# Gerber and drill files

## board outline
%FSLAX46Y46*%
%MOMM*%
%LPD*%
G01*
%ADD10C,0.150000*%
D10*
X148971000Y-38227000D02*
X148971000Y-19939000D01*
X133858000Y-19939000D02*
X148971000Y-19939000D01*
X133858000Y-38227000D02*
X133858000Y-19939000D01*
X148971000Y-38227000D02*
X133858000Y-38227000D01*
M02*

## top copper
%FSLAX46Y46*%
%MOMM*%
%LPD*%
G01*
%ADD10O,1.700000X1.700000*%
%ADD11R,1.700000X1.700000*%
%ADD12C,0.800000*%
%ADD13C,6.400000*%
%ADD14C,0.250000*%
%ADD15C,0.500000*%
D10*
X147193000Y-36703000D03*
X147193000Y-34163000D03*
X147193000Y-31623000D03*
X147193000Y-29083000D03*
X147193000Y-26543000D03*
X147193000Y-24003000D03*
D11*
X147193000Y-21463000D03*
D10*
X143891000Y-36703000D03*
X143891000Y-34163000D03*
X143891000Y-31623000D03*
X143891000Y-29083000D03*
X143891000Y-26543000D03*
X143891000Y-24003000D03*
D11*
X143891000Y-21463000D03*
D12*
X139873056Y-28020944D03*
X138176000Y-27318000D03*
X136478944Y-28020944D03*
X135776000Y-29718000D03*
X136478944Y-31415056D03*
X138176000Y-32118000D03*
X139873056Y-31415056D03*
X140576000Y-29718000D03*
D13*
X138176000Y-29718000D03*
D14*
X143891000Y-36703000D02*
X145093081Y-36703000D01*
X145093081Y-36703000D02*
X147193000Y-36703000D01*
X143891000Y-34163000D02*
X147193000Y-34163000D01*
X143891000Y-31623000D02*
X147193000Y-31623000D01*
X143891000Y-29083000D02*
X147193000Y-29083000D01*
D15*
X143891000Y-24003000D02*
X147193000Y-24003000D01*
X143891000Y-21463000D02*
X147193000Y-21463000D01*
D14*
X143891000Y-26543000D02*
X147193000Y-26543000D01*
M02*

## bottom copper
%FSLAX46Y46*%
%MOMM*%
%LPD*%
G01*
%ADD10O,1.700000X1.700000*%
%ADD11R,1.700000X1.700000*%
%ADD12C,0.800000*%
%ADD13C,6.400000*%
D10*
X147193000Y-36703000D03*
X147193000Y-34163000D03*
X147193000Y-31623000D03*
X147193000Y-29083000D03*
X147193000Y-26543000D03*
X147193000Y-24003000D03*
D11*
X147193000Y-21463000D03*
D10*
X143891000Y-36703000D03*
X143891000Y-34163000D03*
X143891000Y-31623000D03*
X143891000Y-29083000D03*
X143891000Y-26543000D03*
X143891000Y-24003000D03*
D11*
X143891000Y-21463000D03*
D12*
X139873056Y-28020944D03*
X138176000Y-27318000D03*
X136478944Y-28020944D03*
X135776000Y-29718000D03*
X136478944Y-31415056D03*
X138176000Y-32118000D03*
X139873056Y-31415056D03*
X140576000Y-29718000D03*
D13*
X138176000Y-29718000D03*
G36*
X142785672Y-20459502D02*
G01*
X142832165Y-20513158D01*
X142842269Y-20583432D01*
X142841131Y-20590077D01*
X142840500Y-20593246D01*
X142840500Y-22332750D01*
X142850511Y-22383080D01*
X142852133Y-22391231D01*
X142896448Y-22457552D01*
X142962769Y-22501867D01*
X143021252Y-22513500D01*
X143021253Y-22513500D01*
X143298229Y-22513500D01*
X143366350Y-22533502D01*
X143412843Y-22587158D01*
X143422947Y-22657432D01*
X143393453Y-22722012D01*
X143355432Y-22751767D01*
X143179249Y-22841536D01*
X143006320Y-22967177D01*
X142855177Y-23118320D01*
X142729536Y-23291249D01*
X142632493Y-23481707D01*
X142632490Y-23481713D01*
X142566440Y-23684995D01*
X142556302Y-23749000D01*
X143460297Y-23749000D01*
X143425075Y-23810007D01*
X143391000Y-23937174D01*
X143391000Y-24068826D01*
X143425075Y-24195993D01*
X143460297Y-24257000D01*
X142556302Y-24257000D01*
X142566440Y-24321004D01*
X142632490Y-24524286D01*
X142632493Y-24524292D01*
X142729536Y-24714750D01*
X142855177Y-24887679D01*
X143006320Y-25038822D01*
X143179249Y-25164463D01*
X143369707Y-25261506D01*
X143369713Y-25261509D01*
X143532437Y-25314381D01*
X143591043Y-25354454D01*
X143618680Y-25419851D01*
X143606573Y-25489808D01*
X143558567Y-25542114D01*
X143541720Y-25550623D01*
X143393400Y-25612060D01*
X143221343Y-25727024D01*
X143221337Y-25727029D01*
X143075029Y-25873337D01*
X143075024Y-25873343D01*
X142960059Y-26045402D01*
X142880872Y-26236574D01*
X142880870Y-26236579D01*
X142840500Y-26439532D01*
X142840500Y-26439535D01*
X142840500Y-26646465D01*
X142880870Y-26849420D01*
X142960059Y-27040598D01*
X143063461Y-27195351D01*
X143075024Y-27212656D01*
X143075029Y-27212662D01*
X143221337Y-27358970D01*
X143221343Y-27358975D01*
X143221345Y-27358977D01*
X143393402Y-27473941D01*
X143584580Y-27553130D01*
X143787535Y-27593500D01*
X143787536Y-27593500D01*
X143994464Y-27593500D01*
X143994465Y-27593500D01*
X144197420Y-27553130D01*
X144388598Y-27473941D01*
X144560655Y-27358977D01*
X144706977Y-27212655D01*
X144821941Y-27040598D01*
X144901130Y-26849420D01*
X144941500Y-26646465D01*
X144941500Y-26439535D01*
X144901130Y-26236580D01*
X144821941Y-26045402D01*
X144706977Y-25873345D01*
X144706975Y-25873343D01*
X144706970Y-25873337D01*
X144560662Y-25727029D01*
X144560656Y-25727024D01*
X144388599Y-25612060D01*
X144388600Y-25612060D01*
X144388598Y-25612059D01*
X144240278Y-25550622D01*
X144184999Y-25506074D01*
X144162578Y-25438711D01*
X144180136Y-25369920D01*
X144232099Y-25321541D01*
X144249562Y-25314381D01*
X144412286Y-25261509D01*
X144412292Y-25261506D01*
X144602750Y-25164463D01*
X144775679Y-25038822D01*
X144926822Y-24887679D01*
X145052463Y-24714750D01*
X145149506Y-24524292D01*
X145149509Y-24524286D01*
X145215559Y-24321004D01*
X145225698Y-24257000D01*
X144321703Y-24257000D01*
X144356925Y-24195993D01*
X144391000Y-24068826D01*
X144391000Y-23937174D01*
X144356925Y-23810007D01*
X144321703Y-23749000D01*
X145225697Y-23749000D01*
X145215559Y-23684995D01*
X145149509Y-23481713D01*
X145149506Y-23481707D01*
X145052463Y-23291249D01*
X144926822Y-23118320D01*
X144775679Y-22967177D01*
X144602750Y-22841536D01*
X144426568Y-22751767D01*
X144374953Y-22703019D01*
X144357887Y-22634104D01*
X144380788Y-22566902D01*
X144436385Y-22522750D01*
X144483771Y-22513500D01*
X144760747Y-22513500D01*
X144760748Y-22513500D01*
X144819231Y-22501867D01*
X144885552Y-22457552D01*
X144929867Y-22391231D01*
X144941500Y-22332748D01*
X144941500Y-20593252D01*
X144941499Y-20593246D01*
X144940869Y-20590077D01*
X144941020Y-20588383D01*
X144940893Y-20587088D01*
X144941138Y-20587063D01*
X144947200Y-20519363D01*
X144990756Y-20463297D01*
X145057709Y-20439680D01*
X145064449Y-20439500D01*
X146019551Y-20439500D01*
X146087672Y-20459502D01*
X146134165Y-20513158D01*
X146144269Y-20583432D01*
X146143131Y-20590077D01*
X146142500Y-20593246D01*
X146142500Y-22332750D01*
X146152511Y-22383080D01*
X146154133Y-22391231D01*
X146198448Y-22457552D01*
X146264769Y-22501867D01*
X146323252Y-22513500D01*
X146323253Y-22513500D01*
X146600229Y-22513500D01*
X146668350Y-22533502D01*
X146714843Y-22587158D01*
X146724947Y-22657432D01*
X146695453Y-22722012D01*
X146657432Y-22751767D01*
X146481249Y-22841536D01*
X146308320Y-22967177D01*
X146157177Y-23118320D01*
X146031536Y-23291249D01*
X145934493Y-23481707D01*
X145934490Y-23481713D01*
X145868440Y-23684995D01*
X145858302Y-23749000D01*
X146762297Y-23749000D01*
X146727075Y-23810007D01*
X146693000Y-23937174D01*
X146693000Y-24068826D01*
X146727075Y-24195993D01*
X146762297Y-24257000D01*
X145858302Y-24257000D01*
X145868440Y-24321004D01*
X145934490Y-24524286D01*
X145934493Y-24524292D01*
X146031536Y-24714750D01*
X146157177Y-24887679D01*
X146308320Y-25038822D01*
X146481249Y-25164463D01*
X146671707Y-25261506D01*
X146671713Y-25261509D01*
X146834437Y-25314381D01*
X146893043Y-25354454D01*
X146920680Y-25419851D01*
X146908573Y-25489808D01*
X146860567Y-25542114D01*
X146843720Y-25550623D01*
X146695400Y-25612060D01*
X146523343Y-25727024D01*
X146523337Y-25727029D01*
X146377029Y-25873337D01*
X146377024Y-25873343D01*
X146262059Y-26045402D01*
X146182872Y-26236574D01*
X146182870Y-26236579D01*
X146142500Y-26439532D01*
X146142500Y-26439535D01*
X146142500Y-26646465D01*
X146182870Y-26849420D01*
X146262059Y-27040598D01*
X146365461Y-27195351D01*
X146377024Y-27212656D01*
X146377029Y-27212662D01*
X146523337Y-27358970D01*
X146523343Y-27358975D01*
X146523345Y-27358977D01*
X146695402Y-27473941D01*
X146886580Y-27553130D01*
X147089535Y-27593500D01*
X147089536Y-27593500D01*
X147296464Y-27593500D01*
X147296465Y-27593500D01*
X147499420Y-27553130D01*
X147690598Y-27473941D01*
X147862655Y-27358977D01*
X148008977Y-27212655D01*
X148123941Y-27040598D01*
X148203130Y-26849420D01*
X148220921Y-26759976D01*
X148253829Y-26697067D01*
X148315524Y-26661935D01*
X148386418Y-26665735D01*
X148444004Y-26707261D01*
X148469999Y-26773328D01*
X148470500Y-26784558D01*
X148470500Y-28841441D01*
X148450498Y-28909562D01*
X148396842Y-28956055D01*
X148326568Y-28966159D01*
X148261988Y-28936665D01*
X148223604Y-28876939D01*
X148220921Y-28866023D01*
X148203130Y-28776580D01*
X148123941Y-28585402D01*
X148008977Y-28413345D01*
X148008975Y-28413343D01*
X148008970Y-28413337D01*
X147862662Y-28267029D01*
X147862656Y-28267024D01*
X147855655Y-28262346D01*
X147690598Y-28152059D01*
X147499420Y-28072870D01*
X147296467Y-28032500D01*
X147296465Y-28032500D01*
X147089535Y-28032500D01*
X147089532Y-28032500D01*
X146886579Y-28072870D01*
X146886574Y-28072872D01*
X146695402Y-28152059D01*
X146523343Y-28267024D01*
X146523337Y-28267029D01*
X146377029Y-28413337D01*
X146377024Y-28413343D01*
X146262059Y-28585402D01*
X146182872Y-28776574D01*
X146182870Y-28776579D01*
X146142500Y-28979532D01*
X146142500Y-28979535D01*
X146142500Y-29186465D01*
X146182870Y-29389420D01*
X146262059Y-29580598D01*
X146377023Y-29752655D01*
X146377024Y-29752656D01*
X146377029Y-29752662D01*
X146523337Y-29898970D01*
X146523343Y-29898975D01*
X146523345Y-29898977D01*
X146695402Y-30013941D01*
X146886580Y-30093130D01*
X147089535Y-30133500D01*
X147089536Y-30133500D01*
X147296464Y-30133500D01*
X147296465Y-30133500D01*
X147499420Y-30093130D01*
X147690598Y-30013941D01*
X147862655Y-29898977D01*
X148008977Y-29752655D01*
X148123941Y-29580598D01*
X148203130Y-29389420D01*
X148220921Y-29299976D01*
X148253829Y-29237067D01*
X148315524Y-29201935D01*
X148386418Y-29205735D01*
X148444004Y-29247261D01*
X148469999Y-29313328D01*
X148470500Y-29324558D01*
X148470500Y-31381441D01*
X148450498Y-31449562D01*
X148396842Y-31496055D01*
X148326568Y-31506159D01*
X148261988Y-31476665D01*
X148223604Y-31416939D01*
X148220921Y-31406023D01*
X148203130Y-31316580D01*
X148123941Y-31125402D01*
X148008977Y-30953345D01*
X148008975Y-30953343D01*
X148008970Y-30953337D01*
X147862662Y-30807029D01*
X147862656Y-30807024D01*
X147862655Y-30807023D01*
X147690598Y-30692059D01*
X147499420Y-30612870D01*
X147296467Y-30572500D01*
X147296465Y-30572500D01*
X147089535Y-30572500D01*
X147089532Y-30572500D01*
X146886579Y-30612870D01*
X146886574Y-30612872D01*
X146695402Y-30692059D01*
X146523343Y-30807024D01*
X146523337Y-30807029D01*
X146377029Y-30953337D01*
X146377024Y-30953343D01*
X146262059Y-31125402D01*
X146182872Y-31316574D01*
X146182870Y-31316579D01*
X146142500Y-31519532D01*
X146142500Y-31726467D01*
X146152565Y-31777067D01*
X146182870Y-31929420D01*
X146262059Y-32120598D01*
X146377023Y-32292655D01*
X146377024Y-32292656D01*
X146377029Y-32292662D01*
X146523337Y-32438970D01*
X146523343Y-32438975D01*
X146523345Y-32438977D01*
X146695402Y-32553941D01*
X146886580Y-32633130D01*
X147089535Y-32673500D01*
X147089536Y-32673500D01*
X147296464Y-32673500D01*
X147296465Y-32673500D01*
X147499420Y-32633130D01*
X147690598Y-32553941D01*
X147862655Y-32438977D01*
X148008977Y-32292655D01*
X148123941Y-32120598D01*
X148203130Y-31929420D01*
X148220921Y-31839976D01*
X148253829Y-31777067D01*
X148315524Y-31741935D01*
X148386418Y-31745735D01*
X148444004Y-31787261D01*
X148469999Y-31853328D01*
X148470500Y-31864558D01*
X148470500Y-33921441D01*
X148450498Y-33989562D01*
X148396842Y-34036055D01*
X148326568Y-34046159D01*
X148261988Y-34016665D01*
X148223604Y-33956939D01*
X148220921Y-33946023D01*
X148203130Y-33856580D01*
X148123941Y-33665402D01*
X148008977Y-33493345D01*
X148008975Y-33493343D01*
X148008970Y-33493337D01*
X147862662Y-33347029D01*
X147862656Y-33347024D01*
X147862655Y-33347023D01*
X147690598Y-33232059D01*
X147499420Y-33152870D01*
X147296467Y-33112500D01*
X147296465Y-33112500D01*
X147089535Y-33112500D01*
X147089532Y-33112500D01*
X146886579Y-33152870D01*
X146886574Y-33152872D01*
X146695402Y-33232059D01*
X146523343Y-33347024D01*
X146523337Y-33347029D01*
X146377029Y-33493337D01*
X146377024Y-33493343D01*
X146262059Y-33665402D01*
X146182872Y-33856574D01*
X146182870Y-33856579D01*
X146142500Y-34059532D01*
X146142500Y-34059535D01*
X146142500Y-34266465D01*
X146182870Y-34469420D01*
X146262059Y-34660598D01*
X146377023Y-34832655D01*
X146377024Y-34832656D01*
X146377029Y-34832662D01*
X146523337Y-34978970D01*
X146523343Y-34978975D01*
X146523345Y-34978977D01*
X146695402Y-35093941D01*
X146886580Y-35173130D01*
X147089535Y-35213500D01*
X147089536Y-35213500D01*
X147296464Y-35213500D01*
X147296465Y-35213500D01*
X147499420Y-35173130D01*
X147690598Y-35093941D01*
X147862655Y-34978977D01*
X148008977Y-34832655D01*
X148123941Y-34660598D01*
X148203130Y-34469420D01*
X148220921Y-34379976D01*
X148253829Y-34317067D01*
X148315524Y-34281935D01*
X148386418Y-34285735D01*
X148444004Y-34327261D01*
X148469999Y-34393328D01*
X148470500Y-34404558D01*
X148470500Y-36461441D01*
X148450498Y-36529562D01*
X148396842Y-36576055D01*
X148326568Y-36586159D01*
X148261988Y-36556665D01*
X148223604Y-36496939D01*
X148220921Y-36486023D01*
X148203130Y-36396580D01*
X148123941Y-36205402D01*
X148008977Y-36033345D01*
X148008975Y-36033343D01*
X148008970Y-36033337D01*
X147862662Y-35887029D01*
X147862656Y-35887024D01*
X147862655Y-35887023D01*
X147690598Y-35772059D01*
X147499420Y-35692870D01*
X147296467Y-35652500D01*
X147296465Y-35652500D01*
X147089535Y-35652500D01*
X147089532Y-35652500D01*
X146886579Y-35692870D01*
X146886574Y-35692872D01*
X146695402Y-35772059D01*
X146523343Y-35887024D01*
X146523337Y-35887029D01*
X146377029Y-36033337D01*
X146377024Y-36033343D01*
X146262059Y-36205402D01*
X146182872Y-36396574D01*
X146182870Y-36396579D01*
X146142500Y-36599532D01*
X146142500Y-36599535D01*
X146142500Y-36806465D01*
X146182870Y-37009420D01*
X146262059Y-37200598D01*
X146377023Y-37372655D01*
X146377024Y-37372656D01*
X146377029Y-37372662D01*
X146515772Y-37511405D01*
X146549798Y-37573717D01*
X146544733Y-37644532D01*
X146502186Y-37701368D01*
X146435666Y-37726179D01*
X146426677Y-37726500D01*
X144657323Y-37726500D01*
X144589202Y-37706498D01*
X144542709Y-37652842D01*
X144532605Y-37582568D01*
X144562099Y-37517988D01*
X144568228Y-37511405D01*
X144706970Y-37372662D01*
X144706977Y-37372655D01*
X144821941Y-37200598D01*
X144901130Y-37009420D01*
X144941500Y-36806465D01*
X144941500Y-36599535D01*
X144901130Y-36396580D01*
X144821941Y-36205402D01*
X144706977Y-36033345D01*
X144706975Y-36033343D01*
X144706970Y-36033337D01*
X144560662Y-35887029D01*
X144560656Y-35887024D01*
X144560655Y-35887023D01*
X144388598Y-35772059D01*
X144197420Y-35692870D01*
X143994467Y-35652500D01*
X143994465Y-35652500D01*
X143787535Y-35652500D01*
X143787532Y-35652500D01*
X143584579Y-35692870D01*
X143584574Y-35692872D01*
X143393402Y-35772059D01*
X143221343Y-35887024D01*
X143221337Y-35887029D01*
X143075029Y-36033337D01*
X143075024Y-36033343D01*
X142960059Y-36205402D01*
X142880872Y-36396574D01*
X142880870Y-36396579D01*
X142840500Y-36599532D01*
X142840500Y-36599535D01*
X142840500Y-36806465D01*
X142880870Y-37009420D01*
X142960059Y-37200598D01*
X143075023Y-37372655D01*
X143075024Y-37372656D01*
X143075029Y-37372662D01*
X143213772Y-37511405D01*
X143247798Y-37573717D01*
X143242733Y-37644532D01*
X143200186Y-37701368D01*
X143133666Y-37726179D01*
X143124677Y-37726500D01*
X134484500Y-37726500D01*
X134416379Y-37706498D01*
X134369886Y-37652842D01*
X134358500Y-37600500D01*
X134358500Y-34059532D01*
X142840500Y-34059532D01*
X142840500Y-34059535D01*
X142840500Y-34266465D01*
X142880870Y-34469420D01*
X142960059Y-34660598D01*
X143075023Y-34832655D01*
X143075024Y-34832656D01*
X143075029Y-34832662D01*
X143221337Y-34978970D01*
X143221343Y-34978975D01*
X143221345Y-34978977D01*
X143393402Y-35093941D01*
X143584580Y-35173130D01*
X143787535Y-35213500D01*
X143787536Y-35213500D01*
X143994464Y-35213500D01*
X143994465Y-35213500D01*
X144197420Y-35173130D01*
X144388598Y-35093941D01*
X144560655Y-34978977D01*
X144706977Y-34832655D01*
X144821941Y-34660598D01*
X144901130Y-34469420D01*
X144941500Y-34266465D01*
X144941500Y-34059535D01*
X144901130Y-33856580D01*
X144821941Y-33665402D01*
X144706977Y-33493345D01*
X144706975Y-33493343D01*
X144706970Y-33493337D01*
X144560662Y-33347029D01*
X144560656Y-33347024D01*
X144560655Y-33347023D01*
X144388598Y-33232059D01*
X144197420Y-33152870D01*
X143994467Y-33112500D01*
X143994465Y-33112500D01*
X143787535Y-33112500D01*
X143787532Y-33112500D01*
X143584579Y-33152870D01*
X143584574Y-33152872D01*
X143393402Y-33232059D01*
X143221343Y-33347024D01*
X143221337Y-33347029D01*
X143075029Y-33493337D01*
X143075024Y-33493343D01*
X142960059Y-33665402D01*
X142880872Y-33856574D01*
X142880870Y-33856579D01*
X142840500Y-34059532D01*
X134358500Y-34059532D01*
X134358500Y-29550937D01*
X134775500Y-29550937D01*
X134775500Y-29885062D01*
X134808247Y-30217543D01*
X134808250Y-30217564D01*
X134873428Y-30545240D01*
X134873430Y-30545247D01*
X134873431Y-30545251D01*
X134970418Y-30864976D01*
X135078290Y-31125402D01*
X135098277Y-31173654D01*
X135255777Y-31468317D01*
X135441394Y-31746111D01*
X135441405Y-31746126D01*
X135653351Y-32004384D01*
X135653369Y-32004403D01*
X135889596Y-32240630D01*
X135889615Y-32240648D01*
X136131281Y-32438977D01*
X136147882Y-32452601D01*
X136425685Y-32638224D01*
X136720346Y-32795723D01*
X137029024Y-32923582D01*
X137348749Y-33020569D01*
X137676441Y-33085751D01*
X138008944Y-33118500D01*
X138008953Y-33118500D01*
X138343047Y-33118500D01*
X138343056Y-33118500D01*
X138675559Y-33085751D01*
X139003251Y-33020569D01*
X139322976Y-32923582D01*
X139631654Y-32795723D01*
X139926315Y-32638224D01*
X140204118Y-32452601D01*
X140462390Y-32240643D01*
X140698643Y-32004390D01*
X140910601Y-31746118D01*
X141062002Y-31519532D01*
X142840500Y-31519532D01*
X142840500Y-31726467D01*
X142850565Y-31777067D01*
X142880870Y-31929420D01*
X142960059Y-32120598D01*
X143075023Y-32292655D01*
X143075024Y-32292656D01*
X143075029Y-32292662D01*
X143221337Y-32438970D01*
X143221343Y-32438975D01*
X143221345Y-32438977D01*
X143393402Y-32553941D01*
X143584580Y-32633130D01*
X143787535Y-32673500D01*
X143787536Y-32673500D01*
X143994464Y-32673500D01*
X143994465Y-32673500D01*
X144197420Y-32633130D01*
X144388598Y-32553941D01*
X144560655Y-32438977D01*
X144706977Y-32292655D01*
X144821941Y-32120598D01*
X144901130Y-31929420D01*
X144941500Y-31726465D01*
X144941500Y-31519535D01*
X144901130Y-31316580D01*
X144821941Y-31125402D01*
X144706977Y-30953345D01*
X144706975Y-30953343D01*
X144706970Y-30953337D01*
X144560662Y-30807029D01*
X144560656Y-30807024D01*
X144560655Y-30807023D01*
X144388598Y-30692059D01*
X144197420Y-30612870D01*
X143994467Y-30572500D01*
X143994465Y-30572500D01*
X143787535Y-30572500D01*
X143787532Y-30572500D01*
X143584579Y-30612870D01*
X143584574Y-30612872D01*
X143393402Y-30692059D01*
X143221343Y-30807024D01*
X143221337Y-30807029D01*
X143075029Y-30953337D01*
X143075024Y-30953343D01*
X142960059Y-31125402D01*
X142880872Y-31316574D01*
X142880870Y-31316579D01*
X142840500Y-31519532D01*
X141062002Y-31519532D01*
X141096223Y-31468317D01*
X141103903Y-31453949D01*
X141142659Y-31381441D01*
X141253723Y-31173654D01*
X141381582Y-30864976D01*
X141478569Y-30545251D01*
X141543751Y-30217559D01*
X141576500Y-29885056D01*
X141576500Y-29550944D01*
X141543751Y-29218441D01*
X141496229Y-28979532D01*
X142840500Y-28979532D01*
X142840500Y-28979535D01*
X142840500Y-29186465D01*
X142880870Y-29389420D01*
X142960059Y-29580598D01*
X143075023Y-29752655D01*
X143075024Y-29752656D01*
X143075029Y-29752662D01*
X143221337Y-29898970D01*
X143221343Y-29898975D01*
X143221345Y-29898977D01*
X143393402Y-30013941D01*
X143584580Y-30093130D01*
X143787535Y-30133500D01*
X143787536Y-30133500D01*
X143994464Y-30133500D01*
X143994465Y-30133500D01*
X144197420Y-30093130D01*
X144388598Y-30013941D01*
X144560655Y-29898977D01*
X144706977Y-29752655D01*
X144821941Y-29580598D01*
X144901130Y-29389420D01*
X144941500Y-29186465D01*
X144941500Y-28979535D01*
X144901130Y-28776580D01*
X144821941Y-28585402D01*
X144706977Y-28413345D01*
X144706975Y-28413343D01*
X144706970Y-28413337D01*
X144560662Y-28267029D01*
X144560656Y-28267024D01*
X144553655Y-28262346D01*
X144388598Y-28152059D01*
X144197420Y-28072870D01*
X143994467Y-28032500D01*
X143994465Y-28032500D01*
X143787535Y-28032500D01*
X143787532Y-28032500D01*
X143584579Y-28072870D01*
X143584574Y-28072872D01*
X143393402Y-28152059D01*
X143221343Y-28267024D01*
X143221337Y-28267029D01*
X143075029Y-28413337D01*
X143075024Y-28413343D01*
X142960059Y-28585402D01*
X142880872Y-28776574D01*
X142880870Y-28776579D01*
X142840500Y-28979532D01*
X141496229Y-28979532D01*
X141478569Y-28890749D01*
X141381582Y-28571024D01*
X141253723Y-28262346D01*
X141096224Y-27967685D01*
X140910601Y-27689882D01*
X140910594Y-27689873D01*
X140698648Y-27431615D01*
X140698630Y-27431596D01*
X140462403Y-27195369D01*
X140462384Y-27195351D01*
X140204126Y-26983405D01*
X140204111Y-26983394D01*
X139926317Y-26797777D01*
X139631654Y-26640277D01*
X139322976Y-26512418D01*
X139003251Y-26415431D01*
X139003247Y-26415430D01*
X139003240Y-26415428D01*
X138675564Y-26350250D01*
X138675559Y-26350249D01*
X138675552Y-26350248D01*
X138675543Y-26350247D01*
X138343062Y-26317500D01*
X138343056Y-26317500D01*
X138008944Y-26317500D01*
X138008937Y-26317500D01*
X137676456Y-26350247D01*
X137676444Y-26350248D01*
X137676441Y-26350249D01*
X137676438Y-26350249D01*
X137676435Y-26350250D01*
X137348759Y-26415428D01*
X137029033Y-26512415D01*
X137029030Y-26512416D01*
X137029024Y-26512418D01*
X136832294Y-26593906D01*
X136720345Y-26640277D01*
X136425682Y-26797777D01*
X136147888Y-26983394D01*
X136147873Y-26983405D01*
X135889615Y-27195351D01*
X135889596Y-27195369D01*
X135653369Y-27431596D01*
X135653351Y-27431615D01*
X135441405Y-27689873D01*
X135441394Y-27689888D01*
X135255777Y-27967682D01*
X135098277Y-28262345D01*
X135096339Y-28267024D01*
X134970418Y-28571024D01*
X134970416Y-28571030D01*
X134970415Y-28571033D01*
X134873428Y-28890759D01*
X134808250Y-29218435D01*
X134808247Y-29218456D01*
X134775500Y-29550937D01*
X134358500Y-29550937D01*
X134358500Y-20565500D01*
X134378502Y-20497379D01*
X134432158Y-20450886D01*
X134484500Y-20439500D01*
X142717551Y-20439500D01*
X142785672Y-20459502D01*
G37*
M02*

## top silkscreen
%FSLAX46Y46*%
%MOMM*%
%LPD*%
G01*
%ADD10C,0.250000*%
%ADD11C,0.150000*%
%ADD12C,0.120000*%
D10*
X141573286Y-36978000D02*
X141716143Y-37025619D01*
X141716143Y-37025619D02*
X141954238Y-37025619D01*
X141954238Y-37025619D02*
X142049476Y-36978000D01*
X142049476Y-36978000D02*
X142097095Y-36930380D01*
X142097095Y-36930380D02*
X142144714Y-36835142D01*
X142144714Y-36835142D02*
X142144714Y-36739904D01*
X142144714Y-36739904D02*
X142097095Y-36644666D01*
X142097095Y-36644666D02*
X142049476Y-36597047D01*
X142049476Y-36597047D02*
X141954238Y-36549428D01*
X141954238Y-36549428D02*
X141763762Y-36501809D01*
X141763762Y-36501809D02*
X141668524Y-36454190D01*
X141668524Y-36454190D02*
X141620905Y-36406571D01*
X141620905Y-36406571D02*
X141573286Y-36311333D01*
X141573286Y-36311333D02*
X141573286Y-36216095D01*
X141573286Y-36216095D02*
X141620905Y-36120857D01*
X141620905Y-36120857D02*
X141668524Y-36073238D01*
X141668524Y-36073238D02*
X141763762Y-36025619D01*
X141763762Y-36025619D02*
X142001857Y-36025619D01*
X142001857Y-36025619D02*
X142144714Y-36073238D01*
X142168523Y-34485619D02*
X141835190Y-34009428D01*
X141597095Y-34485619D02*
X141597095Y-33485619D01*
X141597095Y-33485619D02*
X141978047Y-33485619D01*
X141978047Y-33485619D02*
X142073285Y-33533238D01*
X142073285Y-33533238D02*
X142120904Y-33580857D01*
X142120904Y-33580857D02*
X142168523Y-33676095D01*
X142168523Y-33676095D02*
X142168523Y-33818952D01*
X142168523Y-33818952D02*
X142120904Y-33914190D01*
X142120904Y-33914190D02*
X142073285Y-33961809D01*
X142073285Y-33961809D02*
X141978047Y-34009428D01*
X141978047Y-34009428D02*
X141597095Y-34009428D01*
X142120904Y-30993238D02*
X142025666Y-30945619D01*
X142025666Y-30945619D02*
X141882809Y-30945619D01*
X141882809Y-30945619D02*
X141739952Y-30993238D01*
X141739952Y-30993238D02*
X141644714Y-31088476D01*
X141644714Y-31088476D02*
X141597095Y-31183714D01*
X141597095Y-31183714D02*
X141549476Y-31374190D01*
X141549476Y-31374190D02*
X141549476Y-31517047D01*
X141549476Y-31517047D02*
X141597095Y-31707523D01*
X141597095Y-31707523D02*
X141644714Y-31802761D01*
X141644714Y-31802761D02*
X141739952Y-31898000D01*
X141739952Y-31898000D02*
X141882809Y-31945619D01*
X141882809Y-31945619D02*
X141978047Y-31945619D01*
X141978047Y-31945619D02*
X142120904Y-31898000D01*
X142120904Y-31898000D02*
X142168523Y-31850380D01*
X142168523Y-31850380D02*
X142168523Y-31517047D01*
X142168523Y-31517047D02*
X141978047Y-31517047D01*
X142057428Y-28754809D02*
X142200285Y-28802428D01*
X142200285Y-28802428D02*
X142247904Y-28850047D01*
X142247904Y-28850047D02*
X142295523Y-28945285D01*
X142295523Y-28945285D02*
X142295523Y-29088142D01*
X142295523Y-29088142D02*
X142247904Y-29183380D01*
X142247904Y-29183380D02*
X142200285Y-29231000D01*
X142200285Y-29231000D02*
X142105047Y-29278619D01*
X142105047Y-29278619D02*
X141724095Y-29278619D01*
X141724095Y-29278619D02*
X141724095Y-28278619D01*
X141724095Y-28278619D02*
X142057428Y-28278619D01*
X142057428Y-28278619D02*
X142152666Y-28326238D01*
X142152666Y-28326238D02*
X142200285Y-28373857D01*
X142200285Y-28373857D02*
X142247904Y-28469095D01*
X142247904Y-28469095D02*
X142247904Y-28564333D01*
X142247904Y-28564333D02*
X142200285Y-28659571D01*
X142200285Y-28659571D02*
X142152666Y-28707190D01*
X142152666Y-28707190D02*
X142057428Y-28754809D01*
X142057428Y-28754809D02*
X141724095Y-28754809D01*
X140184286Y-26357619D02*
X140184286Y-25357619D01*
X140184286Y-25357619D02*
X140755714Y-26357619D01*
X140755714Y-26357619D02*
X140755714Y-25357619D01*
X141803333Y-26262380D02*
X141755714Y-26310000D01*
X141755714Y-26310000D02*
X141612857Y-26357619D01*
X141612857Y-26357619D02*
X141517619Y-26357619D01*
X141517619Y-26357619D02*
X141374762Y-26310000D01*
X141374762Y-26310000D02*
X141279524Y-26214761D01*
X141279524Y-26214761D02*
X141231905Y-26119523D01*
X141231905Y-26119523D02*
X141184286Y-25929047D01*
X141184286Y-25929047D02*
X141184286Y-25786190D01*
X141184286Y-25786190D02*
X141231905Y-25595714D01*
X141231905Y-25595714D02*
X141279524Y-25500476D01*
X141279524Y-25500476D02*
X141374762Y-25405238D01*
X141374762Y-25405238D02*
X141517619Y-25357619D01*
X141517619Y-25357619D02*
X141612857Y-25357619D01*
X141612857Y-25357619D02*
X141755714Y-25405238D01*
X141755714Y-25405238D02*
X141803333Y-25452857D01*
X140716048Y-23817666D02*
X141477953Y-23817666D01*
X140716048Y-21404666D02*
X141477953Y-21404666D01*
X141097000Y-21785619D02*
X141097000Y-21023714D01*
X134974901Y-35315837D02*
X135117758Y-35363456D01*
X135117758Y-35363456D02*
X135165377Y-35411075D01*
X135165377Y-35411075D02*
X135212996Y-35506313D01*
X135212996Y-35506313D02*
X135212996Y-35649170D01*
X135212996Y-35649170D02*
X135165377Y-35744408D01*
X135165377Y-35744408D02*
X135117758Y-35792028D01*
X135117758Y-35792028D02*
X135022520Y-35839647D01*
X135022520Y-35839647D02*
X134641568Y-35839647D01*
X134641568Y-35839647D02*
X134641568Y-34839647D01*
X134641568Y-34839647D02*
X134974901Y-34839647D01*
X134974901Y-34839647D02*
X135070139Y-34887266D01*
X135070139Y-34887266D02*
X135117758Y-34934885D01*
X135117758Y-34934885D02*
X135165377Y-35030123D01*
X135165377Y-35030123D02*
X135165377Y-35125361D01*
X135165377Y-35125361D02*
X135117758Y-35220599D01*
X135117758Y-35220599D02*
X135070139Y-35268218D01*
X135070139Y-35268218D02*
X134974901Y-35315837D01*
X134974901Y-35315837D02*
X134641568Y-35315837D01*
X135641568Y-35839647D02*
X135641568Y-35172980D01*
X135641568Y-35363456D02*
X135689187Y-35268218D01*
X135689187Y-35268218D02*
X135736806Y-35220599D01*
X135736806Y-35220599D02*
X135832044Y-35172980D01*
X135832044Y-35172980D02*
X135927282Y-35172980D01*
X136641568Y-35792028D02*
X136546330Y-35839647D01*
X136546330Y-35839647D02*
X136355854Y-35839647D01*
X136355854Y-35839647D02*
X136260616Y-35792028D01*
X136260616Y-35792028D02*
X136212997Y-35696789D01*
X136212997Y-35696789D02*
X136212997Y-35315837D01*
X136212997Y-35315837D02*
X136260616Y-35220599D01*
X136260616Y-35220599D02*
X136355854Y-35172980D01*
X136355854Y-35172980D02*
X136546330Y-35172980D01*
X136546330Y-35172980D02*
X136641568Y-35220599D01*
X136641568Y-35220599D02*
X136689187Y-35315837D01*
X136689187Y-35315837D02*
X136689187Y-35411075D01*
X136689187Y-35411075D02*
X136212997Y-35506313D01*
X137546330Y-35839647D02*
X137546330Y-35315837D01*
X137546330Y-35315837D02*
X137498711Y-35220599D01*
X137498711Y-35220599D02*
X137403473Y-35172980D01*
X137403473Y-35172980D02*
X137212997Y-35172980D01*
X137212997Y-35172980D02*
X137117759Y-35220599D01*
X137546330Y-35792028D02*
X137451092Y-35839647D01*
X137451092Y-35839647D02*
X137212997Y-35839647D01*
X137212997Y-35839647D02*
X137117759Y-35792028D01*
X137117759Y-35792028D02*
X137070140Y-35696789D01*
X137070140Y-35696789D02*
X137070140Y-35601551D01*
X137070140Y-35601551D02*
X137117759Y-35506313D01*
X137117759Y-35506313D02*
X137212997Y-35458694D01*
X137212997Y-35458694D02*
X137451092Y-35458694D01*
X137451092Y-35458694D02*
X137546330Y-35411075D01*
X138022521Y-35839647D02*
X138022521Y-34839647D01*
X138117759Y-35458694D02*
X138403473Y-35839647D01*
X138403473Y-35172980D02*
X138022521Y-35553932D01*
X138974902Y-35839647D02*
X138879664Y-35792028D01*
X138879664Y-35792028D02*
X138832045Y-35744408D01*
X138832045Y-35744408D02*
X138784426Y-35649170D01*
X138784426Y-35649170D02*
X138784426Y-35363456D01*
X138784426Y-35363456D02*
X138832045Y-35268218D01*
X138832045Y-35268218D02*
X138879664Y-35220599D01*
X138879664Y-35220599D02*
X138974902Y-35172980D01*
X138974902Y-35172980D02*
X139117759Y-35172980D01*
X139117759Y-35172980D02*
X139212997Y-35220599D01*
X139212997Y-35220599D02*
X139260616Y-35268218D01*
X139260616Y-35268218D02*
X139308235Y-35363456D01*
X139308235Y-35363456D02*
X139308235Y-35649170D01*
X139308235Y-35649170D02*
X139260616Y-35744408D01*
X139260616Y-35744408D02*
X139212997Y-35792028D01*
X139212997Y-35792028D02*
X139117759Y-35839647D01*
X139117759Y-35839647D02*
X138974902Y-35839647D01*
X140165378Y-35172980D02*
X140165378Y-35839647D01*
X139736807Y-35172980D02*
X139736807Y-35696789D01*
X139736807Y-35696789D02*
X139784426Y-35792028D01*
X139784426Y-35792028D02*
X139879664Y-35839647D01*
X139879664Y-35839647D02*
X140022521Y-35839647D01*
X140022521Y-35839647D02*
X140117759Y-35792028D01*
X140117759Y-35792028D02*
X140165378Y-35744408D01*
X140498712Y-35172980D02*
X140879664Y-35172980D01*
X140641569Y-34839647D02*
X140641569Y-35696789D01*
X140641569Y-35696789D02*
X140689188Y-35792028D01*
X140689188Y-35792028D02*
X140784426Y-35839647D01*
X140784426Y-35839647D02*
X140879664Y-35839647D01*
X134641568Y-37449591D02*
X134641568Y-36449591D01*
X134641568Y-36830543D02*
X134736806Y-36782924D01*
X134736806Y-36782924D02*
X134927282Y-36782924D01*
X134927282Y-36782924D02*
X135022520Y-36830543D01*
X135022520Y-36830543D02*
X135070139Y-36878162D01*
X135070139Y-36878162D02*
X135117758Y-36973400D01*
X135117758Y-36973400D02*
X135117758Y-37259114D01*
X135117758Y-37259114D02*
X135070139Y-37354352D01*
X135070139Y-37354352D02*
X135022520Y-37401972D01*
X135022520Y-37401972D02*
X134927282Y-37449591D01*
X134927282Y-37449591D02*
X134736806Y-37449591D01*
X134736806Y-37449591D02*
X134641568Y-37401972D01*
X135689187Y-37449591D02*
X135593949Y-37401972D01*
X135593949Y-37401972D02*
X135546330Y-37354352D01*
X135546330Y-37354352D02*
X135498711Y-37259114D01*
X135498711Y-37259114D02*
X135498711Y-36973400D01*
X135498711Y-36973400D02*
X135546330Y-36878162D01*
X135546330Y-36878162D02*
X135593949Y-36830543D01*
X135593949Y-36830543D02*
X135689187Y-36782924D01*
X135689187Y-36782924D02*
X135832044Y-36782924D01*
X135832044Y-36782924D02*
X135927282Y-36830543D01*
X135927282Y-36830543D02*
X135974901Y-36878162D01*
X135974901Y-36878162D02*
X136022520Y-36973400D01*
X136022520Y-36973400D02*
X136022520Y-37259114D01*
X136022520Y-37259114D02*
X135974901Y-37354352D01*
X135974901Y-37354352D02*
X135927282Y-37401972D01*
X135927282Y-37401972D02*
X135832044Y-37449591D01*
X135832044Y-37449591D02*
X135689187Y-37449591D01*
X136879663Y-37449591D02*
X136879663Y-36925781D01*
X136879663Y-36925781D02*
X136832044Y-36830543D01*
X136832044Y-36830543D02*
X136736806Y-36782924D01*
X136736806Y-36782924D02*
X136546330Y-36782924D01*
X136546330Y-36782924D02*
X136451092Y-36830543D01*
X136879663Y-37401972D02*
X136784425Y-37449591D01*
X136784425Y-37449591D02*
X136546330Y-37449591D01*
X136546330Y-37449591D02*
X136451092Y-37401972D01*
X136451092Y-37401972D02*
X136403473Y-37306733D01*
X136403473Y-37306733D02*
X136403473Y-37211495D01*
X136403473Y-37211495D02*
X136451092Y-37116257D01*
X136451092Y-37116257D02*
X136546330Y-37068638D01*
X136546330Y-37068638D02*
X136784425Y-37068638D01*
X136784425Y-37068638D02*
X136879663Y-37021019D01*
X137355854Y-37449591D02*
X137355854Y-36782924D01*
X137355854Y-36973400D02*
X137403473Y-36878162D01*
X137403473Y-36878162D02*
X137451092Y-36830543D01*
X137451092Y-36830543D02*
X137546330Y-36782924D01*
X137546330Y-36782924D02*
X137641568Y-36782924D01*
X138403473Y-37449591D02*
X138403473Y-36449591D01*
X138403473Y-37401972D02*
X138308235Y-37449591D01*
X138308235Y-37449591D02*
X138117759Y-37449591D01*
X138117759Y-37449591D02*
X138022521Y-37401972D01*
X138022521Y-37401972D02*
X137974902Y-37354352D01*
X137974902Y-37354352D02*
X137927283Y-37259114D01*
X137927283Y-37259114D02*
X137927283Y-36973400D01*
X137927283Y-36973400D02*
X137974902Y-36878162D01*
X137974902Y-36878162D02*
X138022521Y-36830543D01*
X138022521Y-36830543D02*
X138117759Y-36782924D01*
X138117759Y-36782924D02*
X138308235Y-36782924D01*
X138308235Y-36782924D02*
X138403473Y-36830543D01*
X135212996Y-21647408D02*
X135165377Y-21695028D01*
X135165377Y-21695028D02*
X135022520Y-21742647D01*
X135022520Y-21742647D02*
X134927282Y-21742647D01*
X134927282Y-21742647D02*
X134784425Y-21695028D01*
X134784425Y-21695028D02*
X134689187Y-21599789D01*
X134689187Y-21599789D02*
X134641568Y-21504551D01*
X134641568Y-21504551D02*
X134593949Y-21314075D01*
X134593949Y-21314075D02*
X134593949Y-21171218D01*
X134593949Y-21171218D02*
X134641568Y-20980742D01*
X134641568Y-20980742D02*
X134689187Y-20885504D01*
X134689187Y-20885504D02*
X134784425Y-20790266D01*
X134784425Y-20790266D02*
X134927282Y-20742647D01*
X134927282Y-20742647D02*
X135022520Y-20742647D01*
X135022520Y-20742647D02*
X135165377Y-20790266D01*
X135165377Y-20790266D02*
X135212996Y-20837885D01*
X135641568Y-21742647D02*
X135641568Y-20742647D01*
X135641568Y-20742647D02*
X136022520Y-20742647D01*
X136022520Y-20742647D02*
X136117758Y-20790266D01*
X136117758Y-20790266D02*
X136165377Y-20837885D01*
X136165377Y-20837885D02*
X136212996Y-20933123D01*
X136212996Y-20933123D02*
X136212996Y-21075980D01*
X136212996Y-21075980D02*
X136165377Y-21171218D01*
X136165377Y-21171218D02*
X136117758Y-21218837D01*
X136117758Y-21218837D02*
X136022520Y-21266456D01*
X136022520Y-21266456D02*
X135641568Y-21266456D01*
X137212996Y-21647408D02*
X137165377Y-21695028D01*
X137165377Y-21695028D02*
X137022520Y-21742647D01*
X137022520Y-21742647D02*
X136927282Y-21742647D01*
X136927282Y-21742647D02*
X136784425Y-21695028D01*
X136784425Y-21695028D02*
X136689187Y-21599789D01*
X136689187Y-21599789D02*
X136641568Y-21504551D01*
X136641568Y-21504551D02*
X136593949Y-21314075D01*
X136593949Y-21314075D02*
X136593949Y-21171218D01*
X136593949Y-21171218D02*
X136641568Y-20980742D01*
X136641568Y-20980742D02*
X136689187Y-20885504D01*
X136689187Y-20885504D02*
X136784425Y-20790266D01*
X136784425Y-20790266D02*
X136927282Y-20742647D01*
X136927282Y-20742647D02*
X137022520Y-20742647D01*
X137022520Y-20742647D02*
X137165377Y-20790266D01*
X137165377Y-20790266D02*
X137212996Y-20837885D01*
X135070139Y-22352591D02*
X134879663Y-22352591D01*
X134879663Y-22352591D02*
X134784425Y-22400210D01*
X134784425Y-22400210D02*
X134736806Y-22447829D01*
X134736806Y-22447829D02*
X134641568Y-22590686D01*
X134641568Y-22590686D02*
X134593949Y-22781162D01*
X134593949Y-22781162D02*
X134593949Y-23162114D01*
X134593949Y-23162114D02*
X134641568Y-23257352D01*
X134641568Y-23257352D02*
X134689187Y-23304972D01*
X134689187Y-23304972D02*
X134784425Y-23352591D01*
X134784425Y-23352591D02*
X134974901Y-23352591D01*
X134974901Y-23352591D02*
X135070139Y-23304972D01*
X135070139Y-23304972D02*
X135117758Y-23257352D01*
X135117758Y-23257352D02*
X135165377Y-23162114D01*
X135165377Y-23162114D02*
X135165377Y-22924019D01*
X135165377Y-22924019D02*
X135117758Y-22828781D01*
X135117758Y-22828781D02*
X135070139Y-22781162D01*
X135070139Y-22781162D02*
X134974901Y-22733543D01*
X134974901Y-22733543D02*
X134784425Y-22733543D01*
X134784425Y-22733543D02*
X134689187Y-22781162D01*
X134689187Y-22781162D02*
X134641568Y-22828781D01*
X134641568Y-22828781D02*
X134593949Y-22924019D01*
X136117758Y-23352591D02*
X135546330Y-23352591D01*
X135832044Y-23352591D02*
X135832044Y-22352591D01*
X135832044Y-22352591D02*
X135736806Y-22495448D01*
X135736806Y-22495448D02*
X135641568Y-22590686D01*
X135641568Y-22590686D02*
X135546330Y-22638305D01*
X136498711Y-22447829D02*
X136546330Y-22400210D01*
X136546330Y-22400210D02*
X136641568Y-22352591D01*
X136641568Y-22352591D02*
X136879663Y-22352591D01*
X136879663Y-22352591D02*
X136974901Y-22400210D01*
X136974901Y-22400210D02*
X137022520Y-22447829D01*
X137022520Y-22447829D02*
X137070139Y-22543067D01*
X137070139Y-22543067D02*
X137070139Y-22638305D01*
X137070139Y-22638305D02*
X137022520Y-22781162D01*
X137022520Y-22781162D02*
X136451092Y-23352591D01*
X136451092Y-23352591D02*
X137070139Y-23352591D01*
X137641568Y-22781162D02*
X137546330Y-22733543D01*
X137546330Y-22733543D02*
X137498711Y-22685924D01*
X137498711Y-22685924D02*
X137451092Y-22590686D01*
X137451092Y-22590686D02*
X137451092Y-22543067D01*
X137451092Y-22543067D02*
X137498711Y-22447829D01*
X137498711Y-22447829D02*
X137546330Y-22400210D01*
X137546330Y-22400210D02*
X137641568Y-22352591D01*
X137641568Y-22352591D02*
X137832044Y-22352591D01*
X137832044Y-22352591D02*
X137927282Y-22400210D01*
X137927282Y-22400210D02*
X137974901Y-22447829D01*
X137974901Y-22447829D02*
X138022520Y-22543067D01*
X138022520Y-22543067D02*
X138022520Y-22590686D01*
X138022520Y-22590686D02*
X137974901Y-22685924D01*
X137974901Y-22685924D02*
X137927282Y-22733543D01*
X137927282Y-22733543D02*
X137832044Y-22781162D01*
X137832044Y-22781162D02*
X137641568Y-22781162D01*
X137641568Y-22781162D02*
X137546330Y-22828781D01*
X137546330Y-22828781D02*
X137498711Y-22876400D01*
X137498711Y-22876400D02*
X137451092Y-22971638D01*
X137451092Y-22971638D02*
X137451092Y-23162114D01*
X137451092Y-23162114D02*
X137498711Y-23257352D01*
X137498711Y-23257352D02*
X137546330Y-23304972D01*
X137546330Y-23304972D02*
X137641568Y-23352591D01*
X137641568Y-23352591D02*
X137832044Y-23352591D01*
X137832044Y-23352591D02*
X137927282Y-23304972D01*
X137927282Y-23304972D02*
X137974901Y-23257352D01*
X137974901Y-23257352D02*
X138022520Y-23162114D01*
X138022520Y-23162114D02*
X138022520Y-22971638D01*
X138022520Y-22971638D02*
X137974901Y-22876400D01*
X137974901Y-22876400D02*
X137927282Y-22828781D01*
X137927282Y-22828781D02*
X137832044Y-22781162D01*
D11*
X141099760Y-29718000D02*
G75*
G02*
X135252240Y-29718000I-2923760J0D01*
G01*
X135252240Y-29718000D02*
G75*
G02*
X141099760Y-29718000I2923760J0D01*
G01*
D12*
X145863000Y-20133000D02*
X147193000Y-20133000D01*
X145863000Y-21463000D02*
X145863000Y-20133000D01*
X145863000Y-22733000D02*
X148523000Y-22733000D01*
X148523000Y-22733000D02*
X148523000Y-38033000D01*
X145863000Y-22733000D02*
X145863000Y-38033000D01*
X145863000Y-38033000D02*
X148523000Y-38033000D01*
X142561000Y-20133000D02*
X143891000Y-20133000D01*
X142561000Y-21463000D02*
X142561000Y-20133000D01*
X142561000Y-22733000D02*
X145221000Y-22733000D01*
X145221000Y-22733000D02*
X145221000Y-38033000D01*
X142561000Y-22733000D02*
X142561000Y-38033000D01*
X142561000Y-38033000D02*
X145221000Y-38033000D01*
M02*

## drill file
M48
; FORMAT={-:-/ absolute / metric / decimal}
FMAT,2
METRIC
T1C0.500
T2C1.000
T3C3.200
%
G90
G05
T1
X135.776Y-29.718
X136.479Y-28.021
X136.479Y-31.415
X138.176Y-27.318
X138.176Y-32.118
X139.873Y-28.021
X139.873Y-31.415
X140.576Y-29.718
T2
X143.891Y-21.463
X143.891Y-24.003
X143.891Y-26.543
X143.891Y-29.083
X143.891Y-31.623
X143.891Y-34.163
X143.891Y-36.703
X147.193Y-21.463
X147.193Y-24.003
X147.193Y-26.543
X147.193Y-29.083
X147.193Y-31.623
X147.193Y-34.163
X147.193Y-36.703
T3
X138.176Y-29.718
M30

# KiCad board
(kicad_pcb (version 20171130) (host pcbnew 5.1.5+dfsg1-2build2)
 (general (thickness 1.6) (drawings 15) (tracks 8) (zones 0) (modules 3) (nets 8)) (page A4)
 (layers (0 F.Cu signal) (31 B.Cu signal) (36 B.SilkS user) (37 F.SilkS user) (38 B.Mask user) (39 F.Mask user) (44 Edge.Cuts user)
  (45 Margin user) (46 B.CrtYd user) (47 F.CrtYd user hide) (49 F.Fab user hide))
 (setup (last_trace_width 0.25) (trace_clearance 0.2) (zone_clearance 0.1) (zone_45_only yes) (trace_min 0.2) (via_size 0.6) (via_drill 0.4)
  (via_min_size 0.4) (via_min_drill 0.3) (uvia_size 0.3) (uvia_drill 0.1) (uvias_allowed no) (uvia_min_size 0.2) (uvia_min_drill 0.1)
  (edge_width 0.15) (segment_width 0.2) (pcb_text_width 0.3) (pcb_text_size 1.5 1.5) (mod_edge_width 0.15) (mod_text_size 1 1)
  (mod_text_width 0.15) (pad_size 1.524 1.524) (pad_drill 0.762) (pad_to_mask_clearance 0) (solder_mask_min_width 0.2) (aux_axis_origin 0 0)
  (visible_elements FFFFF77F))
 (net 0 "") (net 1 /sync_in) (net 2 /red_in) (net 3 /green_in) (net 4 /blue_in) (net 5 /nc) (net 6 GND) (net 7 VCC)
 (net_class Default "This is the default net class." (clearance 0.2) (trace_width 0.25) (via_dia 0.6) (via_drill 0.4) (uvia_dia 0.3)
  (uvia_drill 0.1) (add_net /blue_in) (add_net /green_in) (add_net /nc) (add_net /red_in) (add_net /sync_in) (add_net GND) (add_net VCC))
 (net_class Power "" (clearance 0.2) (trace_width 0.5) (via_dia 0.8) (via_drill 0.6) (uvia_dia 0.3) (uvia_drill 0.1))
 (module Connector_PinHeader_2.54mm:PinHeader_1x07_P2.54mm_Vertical (layer F.Cu) (at 147.193 21.463)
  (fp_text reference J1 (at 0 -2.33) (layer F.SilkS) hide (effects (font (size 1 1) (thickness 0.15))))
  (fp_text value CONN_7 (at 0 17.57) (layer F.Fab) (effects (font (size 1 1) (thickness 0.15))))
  (fp_line (start -1.33 -1.33) (end 0 -1.33) (layer F.SilkS) (width 0.12))
  (fp_line (start -1.33 0) (end -1.33 -1.33) (layer F.SilkS) (width 0.12))
  (fp_line (start -1.33 1.27) (end 1.33 1.27) (layer F.SilkS) (width 0.12))
  (fp_line (start 1.33 1.27) (end 1.33 16.57) (layer F.SilkS) (width 0.12))
  (fp_line (start -1.33 1.27) (end -1.33 16.57) (layer F.SilkS) (width 0.12))
  (fp_line (start -1.33 16.57) (end 1.33 16.57) (layer F.SilkS) (width 0.12))
  (pad 7 thru_hole oval (at 0 15.24) (size 1.7 1.7) (drill 1) (layers *.Cu *.Mask) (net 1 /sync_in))
  (pad 6 thru_hole oval (at 0 12.7) (size 1.7 1.7) (drill 1) (layers *.Cu *.Mask) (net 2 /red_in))
  (pad 5 thru_hole oval (at 0 10.16) (size 1.7 1.7) (drill 1) (layers *.Cu *.Mask) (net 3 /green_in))
  (pad 4 thru_hole oval (at 0 7.62) (size 1.7 1.7) (drill 1) (layers *.Cu *.Mask) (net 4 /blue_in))
  (pad 3 thru_hole oval (at 0 5.08) (size 1.7 1.7) (drill 1) (layers *.Cu *.Mask) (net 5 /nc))
  (pad 2 thru_hole oval (at 0 2.54) (size 1.7 1.7) (drill 1) (layers *.Cu *.Mask) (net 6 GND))
  (pad 1 thru_hole rect (at 0 0) (size 1.7 1.7) (drill 1) (layers *.Cu *.Mask) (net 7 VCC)))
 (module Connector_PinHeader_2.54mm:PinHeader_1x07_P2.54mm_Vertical (layer F.Cu) (at 143.891 21.463)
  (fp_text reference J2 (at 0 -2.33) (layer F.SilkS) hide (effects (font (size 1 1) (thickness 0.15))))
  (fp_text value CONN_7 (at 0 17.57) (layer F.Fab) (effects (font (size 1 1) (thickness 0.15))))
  (fp_line (start -1.33 -1.33) (end 0 -1.33) (layer F.SilkS) (width 0.12))
  (fp_line (start -1.33 0) (end -1.33 -1.33) (layer F.SilkS) (width 0.12))
  (fp_line (start -1.33 1.27) (end 1.33 1.27) (layer F.SilkS) (width 0.12))
  (fp_line (start 1.33 1.27) (end 1.33 16.57) (layer F.SilkS) (width 0.12))
  (fp_line (start -1.33 1.27) (end -1.33 16.57) (layer F.SilkS) (width 0.12))
  (fp_line (start -1.33 16.57) (end 1.33 16.57) (layer F.SilkS) (width 0.12))
  (pad 7 thru_hole oval (at 0 15.24) (size 1.7 1.7) (drill 1) (layers *.Cu *.Mask) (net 1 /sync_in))
  (pad 6 thru_hole oval (at 0 12.7) (size 1.7 1.7) (drill 1) (layers *.Cu *.Mask) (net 2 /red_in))
  (pad 5 thru_hole oval (at 0 10.16) (size 1.7 1.7) (drill 1) (layers *.Cu *.Mask) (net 3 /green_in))
  (pad 4 thru_hole oval (at 0 7.62) (size 1.7 1.7) (drill 1) (layers *.Cu *.Mask) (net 4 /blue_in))
  (pad 3 thru_hole oval (at 0 5.08) (size 1.7 1.7) (drill 1) (layers *.Cu *.Mask) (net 5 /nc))
  (pad 2 thru_hole oval (at 0 2.54) (size 1.7 1.7) (drill 1) (layers *.Cu *.Mask) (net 6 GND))
  (pad 1 thru_hole rect (at 0 0) (size 1.7 1.7) (drill 1) (layers *.Cu *.Mask) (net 7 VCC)))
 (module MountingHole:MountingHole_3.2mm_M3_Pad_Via (layer F.Cu) (at 138.176 29.718)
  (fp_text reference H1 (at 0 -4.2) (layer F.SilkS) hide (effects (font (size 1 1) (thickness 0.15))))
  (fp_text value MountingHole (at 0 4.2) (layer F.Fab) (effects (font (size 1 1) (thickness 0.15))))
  (pad 1 thru_hole circle (at 1.697056 -1.697056) (size 0.8 0.8) (drill 0.5) (layers *.Cu *.Mask))
  (pad 1 thru_hole circle (at 0 -2.4) (size 0.8 0.8) (drill 0.5) (layers *.Cu *.Mask))
  (pad 1 thru_hole circle (at -1.697056 -1.697056) (size 0.8 0.8) (drill 0.5) (layers *.Cu *.Mask))
  (pad 1 thru_hole circle (at -2.4 0) (size 0.8 0.8) (drill 0.5) (layers *.Cu *.Mask))
  (pad 1 thru_hole circle (at -1.697056 1.697056) (size 0.8 0.8) (drill 0.5) (layers *.Cu *.Mask))
  (pad 1 thru_hole circle (at 0 2.4) (size 0.8 0.8) (drill 0.5) (layers *.Cu *.Mask))
  (pad 1 thru_hole circle (at 1.697056 1.697056) (size 0.8 0.8) (drill 0.5) (layers *.Cu *.Mask))
  (pad 1 thru_hole circle (at 2.4 0) (size 0.8 0.8) (drill 0.5) (layers *.Cu *.Mask))
  (pad 1 thru_hole circle (at 0 0) (size 6.4 6.4) (drill 3.2) (layers *.Cu *.Mask)))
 (gr_line (start 148.971 38.227) (end 148.971 19.939) (layer Edge.Cuts) (width 0.15))
 (gr_line (start 133.858 19.939) (end 148.971 19.939) (layer Edge.Cuts) (width 0.15))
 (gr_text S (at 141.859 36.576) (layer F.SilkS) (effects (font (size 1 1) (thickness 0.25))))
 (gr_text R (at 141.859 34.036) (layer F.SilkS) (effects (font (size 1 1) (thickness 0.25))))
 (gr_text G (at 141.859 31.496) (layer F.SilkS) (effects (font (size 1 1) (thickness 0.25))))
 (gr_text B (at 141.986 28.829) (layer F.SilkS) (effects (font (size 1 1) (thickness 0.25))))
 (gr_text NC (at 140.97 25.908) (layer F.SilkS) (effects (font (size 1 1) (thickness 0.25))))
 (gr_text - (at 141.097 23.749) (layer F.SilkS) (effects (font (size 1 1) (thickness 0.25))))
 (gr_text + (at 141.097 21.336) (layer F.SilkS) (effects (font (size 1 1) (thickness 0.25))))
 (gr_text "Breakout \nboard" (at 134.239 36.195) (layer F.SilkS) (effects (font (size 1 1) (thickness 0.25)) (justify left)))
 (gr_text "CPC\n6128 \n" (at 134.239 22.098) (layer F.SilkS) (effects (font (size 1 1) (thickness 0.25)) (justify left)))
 (gr_circle (center 138.176 29.718) (end 139.827 27.305) (layer F.SilkS) (width 0.15))
 (gr_line (start 133.858 38.227) (end 133.858 19.939) (layer Edge.Cuts) (width 0.15))
 (gr_line (start 148.971 38.227) (end 133.858 38.227) (layer Edge.Cuts) (width 0.15))
 (segment (start 143.891 36.703) (end 145.093081 36.703) (width 0.25) (layer F.Cu) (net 1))
 (segment (start 145.093081 36.703) (end 147.193 36.703) (width 0.25) (layer F.Cu) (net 1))
 (segment (start 143.891 34.163) (end 147.193 34.163) (width 0.25) (layer F.Cu) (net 2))
 (segment (start 143.891 31.623) (end 147.193 31.623) (width 0.25) (layer F.Cu) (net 3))
 (segment (start 143.891 29.083) (end 147.193 29.083) (width 0.25) (layer F.Cu) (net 4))
 (segment (start 143.891 24.003) (end 147.193 24.003) (width 0.5) (layer F.Cu) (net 6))
 (segment (start 143.891 21.463) (end 147.193 21.463) (width 0.5) (layer F.Cu) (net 7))
 (segment (start 143.891 26.543) (end 147.193 26.543) (width 0.25) (layer F.Cu) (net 5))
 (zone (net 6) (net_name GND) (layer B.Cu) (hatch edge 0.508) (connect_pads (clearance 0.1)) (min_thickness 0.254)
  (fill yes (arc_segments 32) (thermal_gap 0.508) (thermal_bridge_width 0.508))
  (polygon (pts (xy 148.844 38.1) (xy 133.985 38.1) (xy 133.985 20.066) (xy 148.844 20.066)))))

